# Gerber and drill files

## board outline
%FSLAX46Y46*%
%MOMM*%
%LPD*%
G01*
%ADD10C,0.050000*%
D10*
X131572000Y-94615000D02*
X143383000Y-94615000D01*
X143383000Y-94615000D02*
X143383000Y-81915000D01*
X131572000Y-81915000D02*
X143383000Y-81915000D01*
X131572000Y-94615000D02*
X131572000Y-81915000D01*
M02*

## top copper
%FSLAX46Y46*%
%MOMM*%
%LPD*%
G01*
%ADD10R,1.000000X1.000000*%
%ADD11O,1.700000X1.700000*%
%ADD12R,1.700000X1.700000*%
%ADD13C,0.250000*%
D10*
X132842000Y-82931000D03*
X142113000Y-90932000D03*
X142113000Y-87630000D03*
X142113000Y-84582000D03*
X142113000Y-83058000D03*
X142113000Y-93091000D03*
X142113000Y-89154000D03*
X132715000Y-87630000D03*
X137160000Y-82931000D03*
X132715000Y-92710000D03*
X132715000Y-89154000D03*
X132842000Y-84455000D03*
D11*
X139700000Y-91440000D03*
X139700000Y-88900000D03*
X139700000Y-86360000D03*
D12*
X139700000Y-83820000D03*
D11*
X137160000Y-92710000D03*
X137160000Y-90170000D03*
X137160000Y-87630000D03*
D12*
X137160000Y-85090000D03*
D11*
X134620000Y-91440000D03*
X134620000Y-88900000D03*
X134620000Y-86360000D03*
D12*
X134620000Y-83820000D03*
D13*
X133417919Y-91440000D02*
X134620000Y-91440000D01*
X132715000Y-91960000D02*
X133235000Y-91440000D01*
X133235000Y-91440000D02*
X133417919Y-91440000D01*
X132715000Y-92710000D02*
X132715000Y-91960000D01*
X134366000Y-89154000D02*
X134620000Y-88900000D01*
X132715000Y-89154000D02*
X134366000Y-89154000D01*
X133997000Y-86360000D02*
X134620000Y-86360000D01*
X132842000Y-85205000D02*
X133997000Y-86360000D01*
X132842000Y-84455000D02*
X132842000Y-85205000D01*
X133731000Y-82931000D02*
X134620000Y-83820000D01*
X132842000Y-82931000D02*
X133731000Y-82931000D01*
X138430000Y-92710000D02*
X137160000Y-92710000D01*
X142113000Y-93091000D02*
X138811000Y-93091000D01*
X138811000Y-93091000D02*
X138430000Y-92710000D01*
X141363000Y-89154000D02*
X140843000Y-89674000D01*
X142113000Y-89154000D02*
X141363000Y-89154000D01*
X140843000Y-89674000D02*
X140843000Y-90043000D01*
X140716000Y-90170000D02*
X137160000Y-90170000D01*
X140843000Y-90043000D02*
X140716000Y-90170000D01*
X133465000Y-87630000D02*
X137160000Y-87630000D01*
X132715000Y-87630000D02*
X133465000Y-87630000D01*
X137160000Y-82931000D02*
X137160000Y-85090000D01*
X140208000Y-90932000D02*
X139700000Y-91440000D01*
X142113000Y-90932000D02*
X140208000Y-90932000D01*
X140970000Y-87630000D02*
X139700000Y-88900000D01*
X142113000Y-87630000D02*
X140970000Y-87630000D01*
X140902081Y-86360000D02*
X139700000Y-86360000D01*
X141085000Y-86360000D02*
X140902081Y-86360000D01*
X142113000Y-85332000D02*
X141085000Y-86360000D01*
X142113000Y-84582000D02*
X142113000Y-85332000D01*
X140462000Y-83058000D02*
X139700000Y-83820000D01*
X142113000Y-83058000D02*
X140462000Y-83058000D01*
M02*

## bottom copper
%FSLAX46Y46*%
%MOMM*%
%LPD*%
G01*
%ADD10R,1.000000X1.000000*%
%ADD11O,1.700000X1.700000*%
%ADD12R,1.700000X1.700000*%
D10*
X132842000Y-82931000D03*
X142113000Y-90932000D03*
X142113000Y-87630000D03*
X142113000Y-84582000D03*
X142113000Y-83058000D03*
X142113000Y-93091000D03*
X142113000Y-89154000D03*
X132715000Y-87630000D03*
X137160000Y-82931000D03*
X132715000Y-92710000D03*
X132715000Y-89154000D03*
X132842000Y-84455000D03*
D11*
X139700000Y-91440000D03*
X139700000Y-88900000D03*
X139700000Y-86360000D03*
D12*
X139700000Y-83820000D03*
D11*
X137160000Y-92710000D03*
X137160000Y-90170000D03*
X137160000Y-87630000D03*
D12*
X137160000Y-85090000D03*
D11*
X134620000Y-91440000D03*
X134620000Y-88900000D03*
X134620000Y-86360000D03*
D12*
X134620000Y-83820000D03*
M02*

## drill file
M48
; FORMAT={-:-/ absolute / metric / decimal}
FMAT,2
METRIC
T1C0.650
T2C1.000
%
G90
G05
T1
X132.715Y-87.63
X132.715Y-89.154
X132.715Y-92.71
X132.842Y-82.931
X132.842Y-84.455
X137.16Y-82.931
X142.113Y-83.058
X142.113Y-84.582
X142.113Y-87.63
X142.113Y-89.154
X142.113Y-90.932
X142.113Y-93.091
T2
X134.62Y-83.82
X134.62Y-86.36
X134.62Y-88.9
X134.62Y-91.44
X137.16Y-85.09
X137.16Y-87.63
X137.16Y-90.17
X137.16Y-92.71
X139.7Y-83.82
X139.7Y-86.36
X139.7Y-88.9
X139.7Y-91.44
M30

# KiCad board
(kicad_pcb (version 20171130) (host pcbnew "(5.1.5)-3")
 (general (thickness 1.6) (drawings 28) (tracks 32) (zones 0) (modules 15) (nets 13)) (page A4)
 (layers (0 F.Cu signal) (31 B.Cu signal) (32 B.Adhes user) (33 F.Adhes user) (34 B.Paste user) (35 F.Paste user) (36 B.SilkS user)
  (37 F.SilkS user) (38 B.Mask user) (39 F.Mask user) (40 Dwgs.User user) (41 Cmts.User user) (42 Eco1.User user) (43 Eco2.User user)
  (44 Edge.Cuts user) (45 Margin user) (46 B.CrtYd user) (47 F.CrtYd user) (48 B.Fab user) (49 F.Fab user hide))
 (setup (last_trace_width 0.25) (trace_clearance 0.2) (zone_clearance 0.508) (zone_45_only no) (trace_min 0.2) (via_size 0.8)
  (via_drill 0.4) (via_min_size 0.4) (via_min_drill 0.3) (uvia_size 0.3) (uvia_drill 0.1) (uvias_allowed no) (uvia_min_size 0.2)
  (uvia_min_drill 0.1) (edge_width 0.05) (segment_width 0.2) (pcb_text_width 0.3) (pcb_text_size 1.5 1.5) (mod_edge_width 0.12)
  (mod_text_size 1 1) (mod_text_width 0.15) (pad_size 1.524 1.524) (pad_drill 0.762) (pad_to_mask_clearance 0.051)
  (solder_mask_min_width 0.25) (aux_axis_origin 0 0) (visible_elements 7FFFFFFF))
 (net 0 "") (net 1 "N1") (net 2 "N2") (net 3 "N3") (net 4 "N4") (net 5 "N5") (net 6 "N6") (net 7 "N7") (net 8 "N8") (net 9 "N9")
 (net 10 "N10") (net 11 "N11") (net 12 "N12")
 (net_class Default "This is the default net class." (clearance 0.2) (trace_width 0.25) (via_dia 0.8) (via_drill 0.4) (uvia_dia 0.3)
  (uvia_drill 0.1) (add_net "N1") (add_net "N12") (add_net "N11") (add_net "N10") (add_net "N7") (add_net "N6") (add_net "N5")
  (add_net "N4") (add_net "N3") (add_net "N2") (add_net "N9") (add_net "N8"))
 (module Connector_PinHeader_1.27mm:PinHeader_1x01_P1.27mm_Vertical (layer F.Cu) (at 132.842 82.931)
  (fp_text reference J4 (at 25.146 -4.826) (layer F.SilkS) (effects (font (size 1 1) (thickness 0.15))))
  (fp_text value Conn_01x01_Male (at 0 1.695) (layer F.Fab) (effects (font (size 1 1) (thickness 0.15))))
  (pad 1 thru_hole rect (at 0 0) (size 1 1) (drill 0.65) (layers *.Cu *.Mask) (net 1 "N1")))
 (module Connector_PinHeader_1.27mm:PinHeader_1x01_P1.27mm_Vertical (layer F.Cu) (at 142.113 90.932)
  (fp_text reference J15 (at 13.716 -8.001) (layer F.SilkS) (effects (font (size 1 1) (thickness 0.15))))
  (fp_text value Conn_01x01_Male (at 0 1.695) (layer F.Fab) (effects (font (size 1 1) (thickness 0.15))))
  (pad 1 thru_hole rect (at 0 0) (size 1 1) (drill 0.65) (layers *.Cu *.Mask) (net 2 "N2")))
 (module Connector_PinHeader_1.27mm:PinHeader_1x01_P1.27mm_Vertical (layer F.Cu) (at 142.113 87.63)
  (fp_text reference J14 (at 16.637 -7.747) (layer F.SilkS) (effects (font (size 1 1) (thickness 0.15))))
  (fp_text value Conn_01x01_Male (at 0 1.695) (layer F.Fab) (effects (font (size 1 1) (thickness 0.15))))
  (pad 1 thru_hole rect (at 0 0) (size 1 1) (drill 0.65) (layers *.Cu *.Mask) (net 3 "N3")))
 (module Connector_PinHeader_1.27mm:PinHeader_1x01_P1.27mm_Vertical (layer F.Cu) (at 142.113 84.582)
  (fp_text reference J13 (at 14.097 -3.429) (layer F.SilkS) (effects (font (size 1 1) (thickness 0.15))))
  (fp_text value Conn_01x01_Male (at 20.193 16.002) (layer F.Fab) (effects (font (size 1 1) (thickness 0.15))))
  (pad 1 thru_hole rect (at 0 0) (size 1 1) (drill 0.65) (layers *.Cu *.Mask) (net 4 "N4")))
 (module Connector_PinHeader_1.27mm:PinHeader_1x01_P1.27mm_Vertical (layer F.Cu) (at 142.113 83.058)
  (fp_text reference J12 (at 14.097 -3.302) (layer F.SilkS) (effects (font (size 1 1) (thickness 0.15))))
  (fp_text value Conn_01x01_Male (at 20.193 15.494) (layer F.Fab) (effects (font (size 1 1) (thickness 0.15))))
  (pad 1 thru_hole rect (at 0 0) (size 1 1) (drill 0.65) (layers *.Cu *.Mask) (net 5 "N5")))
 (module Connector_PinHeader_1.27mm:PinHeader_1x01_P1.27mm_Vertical (layer F.Cu) (at 142.113 93.091)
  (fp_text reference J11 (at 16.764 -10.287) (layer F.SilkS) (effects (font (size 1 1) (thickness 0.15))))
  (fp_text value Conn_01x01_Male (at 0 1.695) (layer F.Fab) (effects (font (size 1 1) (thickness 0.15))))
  (pad 1 thru_hole rect (at 0 0) (size 1 1) (drill 0.65) (layers *.Cu *.Mask) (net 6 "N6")))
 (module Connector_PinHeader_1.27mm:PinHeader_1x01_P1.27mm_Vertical (layer F.Cu) (at 142.113 89.154)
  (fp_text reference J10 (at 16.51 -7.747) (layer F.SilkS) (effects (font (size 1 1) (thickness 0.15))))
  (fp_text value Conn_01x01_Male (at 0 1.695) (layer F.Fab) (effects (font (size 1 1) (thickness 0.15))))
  (pad 1 thru_hole rect (at 0 0) (size 1 1) (drill 0.65) (layers *.Cu *.Mask) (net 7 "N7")))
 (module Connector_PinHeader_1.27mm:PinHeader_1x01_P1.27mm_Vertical (layer F.Cu) (at 132.715 87.63)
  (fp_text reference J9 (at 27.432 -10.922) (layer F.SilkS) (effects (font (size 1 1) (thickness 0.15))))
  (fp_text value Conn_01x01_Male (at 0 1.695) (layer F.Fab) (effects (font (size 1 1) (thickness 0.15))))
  (pad 1 thru_hole rect (at 0 0) (size 1 1) (drill 0.65) (layers *.Cu *.Mask) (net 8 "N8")))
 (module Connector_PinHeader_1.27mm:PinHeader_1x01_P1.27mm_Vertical (layer F.Cu) (at 137.16 82.931)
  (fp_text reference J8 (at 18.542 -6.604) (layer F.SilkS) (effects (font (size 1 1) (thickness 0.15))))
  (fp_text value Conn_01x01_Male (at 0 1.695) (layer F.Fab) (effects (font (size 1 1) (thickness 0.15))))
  (pad 1 thru_hole rect (at 0 0) (size 1 1) (drill 0.65) (layers *.Cu *.Mask) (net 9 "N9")))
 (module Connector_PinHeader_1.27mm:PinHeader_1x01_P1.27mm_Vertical (layer F.Cu) (at 132.715 92.71)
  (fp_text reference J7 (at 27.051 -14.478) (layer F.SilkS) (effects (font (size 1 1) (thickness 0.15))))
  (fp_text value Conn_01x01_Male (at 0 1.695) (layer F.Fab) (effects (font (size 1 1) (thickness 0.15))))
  (pad 1 thru_hole rect (at 0 0) (size 1 1) (drill 0.65) (layers *.Cu *.Mask) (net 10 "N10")))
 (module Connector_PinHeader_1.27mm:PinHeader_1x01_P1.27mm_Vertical (layer F.Cu) (at 132.715 89.154)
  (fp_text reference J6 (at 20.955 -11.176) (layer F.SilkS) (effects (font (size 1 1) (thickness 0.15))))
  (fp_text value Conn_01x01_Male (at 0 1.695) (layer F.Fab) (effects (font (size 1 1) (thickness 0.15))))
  (pad 1 thru_hole rect (at 0 0) (size 1 1) (drill 0.65) (layers *.Cu *.Mask) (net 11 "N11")))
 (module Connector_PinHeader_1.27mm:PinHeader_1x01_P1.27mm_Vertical (layer F.Cu) (at 132.842 84.455)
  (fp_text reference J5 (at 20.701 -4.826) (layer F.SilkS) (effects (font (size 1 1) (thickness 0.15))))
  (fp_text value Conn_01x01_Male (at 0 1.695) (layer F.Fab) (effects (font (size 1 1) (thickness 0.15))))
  (pad 1 thru_hole rect (at 0 0) (size 1 1) (drill 0.65) (layers *.Cu *.Mask) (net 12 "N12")))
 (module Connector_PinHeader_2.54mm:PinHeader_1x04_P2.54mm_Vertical (layer F.Cu) (at 139.7 83.82)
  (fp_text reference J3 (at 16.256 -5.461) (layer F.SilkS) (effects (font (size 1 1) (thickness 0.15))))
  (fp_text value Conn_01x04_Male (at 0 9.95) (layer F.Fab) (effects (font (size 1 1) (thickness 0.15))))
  (pad 4 thru_hole oval (at 0 7.62) (size 1.7 1.7) (drill 1) (layers *.Cu *.Mask) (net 2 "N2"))
  (pad 3 thru_hole oval (at 0 5.08) (size 1.7 1.7) (drill 1) (layers *.Cu *.Mask) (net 3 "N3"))
  (pad 2 thru_hole oval (at 0 2.54) (size 1.7 1.7) (drill 1) (layers *.Cu *.Mask) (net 4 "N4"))
  (pad 1 thru_hole rect (at 0 0) (size 1.7 1.7) (drill 1) (layers *.Cu *.Mask) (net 5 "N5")))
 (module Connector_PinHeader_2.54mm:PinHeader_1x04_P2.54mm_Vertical (layer F.Cu) (at 137.16 85.09)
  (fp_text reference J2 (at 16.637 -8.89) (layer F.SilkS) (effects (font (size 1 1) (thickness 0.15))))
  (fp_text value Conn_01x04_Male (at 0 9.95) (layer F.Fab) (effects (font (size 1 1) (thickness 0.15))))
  (pad 4 thru_hole oval (at 0 7.62) (size 1.7 1.7) (drill 1) (layers *.Cu *.Mask) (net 6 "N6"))
  (pad 3 thru_hole oval (at 0 5.08) (size 1.7 1.7) (drill 1) (layers *.Cu *.Mask) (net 7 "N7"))
  (pad 2 thru_hole oval (at 0 2.54) (size 1.7 1.7) (drill 1) (layers *.Cu *.Mask) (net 8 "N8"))
  (pad 1 thru_hole rect (at 0 0) (size 1.7 1.7) (drill 1) (layers *.Cu *.Mask) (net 9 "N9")))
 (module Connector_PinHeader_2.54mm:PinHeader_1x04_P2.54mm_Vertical (layer F.Cu) (at 134.62 83.82)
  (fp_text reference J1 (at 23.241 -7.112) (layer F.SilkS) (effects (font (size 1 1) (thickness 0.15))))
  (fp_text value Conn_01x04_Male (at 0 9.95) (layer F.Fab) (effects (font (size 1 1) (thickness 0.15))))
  (pad 4 thru_hole oval (at 0 7.62) (size 1.7 1.7) (drill 1) (layers *.Cu *.Mask) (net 10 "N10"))
  (pad 3 thru_hole oval (at 0 5.08) (size 1.7 1.7) (drill 1) (layers *.Cu *.Mask) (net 11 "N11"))
  (pad 2 thru_hole oval (at 0 2.54) (size 1.7 1.7) (drill 1) (layers *.Cu *.Mask) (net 12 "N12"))
  (pad 1 thru_hole rect (at 0 0) (size 1.7 1.7) (drill 1) (layers *.Cu *.Mask) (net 1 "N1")))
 (gr_line (start 131.572 94.615) (end 143.383 94.615) (layer Edge.Cuts) (width 0.05))
 (gr_line (start 143.383 94.615) (end 143.383 81.915) (layer Edge.Cuts) (width 0.05))
 (gr_line (start 131.572 81.915) (end 143.383 81.915) (layer Edge.Cuts) (width 0.05))
 (gr_line (start 131.572 94.615) (end 131.572 81.915) (layer Edge.Cuts) (width 0.05))
 (segment (start 133.417919 91.44) (end 134.62 91.44) (width 0.25) (layer F.Cu) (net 10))
 (segment (start 132.715 91.96) (end 133.235 91.44) (width 0.25) (layer F.Cu) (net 10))
 (segment (start 133.235 91.44) (end 133.417919 91.44) (width 0.25) (layer F.Cu) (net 10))
 (segment (start 132.715 92.71) (end 132.715 91.96) (width 0.25) (layer F.Cu) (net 10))
 (segment (start 134.366 89.154) (end 134.62 88.9) (width 0.25) (layer F.Cu) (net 11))
 (segment (start 132.715 89.154) (end 134.366 89.154) (width 0.25) (layer F.Cu) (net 11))
 (segment (start 133.997 86.36) (end 134.62 86.36) (width 0.25) (layer F.Cu) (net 12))
 (segment (start 132.842 85.205) (end 133.997 86.36) (width 0.25) (layer F.Cu) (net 12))
 (segment (start 132.842 84.455) (end 132.842 85.205) (width 0.25) (layer F.Cu) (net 12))
 (segment (start 133.731 82.931) (end 134.62 83.82) (width 0.25) (layer F.Cu) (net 1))
 (segment (start 132.842 82.931) (end 133.731 82.931) (width 0.25) (layer F.Cu) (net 1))
 (segment (start 138.43 92.71) (end 137.16 92.71) (width 0.25) (layer F.Cu) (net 6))
 (segment (start 142.113 93.091) (end 138.811 93.091) (width 0.25) (layer F.Cu) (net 6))
 (segment (start 138.811 93.091) (end 138.43 92.71) (width 0.25) (layer F.Cu) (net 6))
 (segment (start 141.363 89.154) (end 140.843 89.674) (width 0.25) (layer F.Cu) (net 7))
 (segment (start 142.113 89.154) (end 141.363 89.154) (width 0.25) (layer F.Cu) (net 7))
 (segment (start 140.843 89.674) (end 140.843 90.043) (width 0.25) (layer F.Cu) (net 7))
 (segment (start 140.716 90.17) (end 137.16 90.17) (width 0.25) (layer F.Cu) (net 7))
 (segment (start 140.843 90.043) (end 140.716 90.17) (width 0.25) (layer F.Cu) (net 7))
 (segment (start 133.465 87.63) (end 137.16 87.63) (width 0.25) (layer F.Cu) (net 8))
 (segment (start 132.715 87.63) (end 133.465 87.63) (width 0.25) (layer F.Cu) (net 8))
 (segment (start 137.16 82.931) (end 137.16 85.09) (width 0.25) (layer F.Cu) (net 9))
 (segment (start 140.208 90.932) (end 139.7 91.44) (width 0.25) (layer F.Cu) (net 2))
 (segment (start 142.113 90.932) (end 140.208 90.932) (width 0.25) (layer F.Cu) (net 2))
 (segment (start 140.97 87.63) (end 139.7 88.9) (width 0.25) (layer F.Cu) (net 3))
 (segment (start 142.113 87.63) (end 140.97 87.63) (width 0.25) (layer F.Cu) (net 3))
 (segment (start 140.902081 86.36) (end 139.7 86.36) (width 0.25) (layer F.Cu) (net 4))
 (segment (start 141.085 86.36) (end 140.902081 86.36) (width 0.25) (layer F.Cu) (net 4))
 (segment (start 142.113 85.332) (end 141.085 86.36) (width 0.25) (layer F.Cu) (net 4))
 (segment (start 142.113 84.582) (end 142.113 85.332) (width 0.25) (layer F.Cu) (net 4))
 (segment (start 140.462 83.058) (end 139.7 83.82) (width 0.25) (layer F.Cu) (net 5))
 (segment (start 142.113 83.058) (end 140.462 83.058) (width 0.25) (layer F.Cu) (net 5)))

